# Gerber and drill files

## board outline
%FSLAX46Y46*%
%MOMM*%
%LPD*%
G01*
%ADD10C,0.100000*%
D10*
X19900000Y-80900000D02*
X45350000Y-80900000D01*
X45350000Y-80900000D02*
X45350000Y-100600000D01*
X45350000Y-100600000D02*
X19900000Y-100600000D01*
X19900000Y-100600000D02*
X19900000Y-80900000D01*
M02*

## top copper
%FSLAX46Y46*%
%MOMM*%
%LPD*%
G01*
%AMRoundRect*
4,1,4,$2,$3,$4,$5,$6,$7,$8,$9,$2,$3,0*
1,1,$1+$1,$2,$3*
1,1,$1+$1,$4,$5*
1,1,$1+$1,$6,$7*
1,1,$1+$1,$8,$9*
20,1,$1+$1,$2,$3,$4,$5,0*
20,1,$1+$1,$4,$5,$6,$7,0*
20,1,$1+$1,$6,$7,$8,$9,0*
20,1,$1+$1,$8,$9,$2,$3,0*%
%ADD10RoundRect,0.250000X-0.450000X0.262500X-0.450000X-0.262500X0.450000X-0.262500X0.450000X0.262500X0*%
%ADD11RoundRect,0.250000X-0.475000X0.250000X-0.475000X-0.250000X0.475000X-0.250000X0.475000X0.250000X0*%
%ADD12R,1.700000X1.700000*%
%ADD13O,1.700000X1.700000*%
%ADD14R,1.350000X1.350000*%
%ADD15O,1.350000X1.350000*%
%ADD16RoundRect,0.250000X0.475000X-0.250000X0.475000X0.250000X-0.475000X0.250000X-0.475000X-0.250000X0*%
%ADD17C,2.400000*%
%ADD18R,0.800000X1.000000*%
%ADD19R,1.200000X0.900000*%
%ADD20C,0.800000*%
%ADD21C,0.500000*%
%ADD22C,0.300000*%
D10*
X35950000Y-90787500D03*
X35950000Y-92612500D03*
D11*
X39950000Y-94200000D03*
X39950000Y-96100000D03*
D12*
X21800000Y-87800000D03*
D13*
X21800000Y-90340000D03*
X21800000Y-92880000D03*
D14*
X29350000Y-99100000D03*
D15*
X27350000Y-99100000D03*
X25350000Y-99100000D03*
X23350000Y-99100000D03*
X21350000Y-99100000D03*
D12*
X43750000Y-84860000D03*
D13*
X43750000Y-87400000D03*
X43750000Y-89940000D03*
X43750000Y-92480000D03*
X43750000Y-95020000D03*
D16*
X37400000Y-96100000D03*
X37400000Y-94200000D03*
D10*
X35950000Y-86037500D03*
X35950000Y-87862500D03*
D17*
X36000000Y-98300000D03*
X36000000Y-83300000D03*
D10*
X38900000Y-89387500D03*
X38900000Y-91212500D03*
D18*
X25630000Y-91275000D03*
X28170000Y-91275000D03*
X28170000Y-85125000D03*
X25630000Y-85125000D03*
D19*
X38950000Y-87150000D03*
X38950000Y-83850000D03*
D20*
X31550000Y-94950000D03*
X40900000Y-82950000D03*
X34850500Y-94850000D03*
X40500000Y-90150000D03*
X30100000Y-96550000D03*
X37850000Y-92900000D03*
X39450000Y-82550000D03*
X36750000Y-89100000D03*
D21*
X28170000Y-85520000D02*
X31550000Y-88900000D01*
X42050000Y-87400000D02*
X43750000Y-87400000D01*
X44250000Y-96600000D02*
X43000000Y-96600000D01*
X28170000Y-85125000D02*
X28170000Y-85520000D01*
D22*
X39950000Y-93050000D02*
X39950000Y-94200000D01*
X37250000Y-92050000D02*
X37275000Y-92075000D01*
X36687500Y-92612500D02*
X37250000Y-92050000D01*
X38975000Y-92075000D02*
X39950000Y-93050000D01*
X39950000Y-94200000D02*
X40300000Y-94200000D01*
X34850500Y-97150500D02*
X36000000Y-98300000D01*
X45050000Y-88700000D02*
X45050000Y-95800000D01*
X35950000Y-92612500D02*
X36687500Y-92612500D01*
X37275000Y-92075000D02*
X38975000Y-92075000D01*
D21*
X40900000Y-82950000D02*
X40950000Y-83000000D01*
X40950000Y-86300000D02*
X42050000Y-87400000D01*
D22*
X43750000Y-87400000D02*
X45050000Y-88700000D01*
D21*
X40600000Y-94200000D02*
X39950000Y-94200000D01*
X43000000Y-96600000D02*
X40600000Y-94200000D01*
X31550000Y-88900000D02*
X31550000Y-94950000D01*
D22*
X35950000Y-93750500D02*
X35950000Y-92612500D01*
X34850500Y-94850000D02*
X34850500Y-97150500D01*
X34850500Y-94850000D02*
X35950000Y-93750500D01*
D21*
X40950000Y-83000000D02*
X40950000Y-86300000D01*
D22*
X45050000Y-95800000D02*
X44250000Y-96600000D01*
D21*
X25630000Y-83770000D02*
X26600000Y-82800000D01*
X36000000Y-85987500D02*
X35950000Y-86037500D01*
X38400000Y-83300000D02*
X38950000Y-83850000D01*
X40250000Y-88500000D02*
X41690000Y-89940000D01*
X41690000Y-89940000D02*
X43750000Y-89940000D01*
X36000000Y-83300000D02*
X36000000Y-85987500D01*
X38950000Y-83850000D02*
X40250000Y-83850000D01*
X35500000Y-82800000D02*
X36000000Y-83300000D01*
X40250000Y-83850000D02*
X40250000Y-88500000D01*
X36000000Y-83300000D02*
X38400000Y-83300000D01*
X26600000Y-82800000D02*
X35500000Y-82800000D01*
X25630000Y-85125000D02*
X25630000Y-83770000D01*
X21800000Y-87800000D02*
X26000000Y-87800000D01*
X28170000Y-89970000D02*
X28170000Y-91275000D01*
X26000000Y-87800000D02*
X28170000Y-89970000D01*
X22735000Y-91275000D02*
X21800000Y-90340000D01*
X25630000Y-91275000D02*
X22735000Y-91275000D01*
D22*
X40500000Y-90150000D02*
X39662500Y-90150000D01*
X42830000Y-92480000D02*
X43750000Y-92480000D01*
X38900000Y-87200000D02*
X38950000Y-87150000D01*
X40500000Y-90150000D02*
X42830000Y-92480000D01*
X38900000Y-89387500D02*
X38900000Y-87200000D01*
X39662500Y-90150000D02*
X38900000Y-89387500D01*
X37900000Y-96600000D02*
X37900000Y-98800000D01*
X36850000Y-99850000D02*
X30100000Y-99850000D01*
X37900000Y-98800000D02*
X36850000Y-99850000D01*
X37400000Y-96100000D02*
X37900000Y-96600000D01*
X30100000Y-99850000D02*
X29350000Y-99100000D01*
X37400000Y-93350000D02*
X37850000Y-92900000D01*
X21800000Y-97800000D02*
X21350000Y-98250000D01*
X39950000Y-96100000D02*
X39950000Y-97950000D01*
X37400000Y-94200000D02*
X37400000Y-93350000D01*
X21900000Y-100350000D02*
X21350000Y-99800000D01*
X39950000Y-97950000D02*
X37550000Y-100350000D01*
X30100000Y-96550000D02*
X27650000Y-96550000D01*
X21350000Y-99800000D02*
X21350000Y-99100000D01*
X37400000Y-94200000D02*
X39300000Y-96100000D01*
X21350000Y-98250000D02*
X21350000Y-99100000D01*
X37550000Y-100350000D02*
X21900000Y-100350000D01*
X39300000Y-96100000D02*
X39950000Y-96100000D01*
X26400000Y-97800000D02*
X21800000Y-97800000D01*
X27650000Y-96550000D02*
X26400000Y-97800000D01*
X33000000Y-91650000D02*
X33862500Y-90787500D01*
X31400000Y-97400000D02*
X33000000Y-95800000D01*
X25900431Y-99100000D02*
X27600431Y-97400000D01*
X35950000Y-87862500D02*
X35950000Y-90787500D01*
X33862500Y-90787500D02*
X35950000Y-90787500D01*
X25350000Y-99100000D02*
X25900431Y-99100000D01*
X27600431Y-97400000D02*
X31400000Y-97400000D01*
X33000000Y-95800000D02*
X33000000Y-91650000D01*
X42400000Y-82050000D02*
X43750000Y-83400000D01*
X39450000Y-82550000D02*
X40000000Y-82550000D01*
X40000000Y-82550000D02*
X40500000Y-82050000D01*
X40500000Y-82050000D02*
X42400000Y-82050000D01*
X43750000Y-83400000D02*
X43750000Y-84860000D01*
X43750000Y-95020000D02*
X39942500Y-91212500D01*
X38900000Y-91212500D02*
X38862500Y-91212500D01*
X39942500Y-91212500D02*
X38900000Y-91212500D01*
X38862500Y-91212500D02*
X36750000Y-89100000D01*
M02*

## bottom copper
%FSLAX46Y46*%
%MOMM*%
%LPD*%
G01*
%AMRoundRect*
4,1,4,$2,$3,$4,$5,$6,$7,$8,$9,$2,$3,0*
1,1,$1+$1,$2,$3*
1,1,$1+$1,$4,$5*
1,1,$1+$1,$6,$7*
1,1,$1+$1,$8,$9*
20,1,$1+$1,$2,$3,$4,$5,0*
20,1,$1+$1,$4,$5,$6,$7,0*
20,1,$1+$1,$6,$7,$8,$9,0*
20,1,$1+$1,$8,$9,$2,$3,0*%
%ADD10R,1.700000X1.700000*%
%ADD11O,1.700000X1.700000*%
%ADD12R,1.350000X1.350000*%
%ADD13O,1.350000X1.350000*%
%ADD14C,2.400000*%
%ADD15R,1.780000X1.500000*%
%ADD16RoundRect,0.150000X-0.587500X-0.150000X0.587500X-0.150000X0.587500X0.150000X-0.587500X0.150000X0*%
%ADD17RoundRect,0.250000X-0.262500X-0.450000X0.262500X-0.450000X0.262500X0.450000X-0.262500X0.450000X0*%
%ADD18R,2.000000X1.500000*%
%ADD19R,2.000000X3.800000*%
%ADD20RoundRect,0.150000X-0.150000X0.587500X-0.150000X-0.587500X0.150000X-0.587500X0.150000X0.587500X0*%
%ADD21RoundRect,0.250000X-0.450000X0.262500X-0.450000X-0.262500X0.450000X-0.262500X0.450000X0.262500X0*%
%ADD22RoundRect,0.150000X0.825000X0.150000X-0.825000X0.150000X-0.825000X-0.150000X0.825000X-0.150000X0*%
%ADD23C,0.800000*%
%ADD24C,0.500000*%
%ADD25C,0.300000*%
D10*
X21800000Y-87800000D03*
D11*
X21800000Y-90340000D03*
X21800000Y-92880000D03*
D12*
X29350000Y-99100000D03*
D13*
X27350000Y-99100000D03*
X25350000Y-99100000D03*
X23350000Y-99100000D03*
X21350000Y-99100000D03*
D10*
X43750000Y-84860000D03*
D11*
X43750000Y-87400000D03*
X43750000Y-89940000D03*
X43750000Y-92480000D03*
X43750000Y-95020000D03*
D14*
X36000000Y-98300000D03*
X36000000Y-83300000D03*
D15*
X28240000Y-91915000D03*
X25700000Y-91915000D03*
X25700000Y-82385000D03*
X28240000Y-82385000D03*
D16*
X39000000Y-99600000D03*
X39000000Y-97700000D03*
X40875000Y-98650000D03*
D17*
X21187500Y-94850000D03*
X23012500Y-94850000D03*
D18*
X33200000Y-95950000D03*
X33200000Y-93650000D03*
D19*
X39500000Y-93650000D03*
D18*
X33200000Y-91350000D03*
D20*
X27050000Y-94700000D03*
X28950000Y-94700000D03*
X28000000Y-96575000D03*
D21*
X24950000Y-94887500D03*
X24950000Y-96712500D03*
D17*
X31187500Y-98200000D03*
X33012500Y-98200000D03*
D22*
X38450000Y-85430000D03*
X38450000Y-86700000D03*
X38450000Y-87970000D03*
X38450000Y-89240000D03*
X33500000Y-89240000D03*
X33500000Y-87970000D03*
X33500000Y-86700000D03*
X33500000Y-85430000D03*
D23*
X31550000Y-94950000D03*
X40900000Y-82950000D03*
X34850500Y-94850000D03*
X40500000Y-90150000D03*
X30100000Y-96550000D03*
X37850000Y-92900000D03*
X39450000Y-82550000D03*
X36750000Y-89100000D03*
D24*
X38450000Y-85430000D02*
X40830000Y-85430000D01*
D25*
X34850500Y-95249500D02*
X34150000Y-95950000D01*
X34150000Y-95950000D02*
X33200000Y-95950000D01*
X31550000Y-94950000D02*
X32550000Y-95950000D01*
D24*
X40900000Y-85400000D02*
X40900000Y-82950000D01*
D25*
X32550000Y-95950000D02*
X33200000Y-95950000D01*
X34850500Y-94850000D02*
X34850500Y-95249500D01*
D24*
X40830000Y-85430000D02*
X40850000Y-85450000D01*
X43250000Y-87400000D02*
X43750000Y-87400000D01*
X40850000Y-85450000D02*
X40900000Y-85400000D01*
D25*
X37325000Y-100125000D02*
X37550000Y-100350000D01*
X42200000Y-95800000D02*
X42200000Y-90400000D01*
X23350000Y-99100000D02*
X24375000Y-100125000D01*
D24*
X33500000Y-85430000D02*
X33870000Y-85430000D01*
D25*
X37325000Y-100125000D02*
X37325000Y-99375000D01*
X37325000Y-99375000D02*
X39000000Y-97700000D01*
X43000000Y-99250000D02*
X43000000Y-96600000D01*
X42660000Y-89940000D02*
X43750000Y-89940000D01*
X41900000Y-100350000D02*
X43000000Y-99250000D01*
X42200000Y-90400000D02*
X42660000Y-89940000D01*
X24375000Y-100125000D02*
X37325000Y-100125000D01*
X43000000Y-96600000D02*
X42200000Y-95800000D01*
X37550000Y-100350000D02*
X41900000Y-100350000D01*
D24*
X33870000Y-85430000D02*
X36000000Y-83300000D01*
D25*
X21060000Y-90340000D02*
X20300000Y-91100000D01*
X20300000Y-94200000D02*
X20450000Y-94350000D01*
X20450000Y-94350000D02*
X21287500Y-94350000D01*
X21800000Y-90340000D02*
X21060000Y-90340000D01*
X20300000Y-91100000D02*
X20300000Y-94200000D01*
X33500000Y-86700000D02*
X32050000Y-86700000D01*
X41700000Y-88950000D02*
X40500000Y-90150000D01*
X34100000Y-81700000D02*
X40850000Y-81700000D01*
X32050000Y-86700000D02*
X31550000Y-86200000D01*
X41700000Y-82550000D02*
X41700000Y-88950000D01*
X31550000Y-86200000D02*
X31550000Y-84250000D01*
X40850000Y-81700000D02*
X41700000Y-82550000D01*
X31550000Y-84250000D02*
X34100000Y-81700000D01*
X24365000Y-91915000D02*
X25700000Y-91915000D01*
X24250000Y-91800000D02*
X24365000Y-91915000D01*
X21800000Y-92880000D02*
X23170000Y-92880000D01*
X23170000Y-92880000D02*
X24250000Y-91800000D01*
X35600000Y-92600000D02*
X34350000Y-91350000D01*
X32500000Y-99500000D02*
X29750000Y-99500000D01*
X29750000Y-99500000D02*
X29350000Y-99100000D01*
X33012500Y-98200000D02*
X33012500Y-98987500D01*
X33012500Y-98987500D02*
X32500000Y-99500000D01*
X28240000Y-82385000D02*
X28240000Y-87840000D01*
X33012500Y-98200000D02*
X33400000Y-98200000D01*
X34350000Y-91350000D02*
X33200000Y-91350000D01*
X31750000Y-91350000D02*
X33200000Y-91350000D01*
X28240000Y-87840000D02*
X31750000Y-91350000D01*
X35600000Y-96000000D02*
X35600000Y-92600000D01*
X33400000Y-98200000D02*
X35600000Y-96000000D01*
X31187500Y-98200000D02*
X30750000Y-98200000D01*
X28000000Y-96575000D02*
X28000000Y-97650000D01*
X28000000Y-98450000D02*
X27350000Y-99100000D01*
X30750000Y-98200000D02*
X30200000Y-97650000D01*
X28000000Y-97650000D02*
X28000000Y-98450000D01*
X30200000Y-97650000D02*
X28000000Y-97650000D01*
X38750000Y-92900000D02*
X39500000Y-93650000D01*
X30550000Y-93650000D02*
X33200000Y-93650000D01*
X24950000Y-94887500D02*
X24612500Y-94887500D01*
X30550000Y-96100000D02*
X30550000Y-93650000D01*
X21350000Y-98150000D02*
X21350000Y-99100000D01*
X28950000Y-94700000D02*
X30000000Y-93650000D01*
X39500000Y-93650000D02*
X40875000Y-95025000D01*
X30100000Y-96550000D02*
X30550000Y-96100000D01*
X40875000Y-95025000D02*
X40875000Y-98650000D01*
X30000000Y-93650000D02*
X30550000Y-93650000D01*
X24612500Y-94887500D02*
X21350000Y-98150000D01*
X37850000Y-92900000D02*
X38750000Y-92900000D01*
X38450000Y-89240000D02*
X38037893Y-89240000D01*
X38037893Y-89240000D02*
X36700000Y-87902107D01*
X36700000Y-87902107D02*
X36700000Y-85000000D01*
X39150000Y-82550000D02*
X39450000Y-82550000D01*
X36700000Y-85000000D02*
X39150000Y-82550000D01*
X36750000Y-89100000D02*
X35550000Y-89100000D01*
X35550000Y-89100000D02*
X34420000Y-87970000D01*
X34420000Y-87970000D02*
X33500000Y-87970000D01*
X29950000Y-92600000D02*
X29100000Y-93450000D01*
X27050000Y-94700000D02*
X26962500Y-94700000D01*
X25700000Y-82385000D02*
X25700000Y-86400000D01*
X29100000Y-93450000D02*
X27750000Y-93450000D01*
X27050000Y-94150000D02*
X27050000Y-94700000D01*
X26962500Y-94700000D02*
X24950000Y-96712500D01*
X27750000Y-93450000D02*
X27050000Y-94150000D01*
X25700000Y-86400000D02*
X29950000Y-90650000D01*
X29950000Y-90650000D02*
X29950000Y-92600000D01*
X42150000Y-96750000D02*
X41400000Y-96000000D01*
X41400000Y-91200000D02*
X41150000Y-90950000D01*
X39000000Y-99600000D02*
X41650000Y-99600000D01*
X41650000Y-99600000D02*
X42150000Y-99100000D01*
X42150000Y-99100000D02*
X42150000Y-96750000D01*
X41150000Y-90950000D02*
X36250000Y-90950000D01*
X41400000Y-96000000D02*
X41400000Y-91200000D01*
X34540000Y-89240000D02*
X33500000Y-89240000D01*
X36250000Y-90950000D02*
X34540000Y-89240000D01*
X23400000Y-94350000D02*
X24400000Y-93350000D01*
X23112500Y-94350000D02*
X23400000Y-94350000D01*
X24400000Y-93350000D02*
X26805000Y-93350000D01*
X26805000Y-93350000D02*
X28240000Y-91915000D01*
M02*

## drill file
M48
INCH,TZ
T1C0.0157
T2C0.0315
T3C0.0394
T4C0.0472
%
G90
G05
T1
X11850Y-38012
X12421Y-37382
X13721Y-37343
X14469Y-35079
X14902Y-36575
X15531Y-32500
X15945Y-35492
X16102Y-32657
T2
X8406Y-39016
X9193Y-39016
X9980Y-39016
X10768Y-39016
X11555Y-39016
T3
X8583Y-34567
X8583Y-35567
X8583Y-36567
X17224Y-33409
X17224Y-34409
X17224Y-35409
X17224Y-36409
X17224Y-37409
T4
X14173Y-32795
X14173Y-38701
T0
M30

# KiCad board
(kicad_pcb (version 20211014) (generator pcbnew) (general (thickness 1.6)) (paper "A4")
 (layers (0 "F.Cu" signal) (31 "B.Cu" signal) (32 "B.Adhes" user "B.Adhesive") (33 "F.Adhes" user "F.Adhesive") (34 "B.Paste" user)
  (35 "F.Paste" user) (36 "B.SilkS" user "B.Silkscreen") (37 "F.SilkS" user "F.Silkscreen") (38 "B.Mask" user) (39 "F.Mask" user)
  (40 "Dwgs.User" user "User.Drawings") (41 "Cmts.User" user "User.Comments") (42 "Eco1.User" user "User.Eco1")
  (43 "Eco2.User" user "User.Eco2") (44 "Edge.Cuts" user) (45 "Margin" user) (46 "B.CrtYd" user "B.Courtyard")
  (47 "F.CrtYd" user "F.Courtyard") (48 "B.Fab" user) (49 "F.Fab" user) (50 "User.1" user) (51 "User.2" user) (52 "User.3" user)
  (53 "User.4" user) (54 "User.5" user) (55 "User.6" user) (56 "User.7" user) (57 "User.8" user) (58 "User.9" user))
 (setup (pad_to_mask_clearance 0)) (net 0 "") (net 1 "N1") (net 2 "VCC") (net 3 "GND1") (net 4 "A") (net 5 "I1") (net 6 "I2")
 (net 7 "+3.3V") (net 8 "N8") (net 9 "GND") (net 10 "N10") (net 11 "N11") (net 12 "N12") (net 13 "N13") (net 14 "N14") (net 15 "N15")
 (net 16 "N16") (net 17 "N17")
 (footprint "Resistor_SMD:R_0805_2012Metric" (layer "F.Cu") (at 35.95 91.7 -90)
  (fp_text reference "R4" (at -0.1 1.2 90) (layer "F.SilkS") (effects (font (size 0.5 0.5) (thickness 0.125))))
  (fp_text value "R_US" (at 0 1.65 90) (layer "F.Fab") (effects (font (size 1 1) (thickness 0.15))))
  (pad "1" smd roundrect (at -0.9125 0 270) (size 1.025 1.4) (layers "F.Cu" "F.Paste" "F.Mask") (roundrect_rratio 0.243902439) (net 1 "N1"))
  (pad "2" smd roundrect (at 0.9125 0 270) (size 1.025 1.4) (layers "F.Cu" "F.Paste" "F.Mask") (roundrect_rratio 0.243902439) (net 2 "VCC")))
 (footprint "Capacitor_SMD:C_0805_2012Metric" (layer "F.Cu") (at 39.95 95.15 -90)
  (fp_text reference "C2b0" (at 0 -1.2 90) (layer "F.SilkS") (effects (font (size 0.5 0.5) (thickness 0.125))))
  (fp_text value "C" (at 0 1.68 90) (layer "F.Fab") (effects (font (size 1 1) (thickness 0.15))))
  (pad "1" smd roundrect (at -0.95 0 270) (size 1 1.45) (layers "F.Cu" "F.Paste" "F.Mask") (roundrect_rratio 0.25) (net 2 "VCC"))
  (pad "2" smd roundrect (at 0.95 0 270) (size 1 1.45) (layers "F.Cu" "F.Paste" "F.Mask") (roundrect_rratio 0.25) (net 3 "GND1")))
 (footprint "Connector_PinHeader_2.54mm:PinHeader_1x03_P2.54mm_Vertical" (layer "F.Cu") (at 21.8 87.8)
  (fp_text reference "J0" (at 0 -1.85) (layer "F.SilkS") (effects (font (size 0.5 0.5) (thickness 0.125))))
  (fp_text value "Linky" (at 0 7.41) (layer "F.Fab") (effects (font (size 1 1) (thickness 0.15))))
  (pad "1" thru_hole rect (at 0 0) (size 1.7 1.7) (drill 1) (layers *.Cu *.Mask) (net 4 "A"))
  (pad "2" thru_hole oval (at 0 2.54) (size 1.7 1.7) (drill 1) (layers *.Cu *.Mask) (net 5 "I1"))
  (pad "3" thru_hole oval (at 0 5.08) (size 1.7 1.7) (drill 1) (layers *.Cu *.Mask) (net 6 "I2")))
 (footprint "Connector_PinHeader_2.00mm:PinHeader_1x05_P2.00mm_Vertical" (layer "F.Cu") (at 29.35 99.1 -90)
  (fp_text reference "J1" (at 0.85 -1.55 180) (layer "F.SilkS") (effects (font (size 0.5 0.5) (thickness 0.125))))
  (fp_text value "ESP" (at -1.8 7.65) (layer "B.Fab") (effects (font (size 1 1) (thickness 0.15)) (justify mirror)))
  (pad "1" thru_hole rect (at 0 0 270) (size 1.35 1.35) (drill 0.8) (layers *.Cu *.Mask) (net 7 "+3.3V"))
  (pad "2" thru_hole oval (at 0 2 270) (size 1.35 1.35) (drill 0.8) (layers *.Cu *.Mask) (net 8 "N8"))
  (pad "3" thru_hole oval (at 0 4 270) (size 1.35 1.35) (drill 0.8) (layers *.Cu *.Mask) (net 1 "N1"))
  (pad "4" thru_hole oval (at 0 6 270) (size 1.35 1.35) (drill 0.8) (layers *.Cu *.Mask) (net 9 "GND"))
  (pad "5" thru_hole oval (at 0 8 270) (size 1.35 1.35) (drill 0.8) (layers *.Cu *.Mask) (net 3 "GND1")))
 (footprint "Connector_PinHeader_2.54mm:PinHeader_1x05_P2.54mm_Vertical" (layer "F.Cu") (at 43.75 84.86)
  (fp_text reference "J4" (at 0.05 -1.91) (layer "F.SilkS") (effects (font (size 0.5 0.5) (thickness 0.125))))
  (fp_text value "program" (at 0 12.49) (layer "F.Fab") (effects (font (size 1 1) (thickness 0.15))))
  (pad "1" thru_hole rect (at 0 0) (size 1.7 1.7) (drill 1) (layers *.Cu *.Mask) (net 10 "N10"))
  (pad "2" thru_hole oval (at 0 2.54) (size 1.7 1.7) (drill 1) (layers *.Cu *.Mask) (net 2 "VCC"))
  (pad "3" thru_hole oval (at 0 5.08) (size 1.7 1.7) (drill 1) (layers *.Cu *.Mask) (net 9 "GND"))
  (pad "4" thru_hole oval (at 0 7.62) (size 1.7 1.7) (drill 1) (layers *.Cu *.Mask) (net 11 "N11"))
  (pad "5" thru_hole oval (at 0 10.16) (size 1.7 1.7) (drill 1) (layers *.Cu *.Mask) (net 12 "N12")))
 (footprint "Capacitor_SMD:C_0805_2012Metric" (layer "F.Cu") (at 37.4 95.15 90)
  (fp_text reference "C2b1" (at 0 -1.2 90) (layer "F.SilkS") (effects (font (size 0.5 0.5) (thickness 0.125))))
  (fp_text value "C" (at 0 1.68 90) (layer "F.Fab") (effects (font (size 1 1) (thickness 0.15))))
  (pad "1" smd roundrect (at -0.95 0 90) (size 1 1.45) (layers "F.Cu" "F.Paste" "F.Mask") (roundrect_rratio 0.25) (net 7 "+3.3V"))
  (pad "2" smd roundrect (at 0.95 0 90) (size 1 1.45) (layers "F.Cu" "F.Paste" "F.Mask") (roundrect_rratio 0.25) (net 3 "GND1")))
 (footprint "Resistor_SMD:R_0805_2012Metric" (layer "F.Cu") (at 35.95 86.95 -90)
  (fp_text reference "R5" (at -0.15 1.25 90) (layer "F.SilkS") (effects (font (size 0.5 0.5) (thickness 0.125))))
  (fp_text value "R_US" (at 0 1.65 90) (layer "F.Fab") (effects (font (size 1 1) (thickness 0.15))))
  (pad "1" smd roundrect (at -0.9125 0 270) (size 1.025 1.4) (layers "F.Cu" "F.Paste" "F.Mask") (roundrect_rratio 0.243902439) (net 9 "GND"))
  (pad "2" smd roundrect (at 0.9125 0 270) (size 1.025 1.4) (layers "F.Cu" "F.Paste" "F.Mask") (roundrect_rratio 0.243902439) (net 1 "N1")))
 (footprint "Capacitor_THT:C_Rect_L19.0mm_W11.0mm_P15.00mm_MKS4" (layer "F.Cu") (at 36 98.3 90)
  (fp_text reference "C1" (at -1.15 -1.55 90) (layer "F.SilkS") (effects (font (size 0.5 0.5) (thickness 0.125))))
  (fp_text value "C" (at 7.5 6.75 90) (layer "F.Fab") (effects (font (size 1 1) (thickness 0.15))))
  (pad "1" thru_hole circle (at 0 0 90) (size 2.4 2.4) (drill 1.2) (layers *.Cu *.Mask) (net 2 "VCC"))
  (pad "2" thru_hole circle (at 15 0 90) (size 2.4 2.4) (drill 1.2) (layers *.Cu *.Mask) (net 9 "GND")))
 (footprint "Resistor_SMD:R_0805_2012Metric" (layer "F.Cu") (at 38.9 90.3 -90)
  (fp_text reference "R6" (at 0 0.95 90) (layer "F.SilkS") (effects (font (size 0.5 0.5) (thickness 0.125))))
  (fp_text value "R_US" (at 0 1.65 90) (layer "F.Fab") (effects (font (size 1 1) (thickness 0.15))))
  (pad "1" smd roundrect (at -0.9125 0 270) (size 1.025 1.4) (layers "F.Cu" "F.Paste" "F.Mask") (roundrect_rratio 0.243902439)
   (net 11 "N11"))
  (pad "2" smd roundrect (at 0.9125 0 270) (size 1.025 1.4) (layers "F.Cu" "F.Paste" "F.Mask") (roundrect_rratio 0.243902439) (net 12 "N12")))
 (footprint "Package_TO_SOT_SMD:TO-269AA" (layer "F.Cu") (at 26.9 88.2 90)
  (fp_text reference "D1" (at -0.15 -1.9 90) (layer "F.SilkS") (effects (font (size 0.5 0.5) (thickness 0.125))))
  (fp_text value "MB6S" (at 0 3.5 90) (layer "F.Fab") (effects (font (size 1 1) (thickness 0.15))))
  (pad "1" smd rect (at -3.075 -1.27 90) (size 1 0.8) (layers "F.Cu" "F.Paste" "F.Mask") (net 5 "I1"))
  (pad "2" smd rect (at -3.075 1.27 90) (size 1 0.8) (layers "F.Cu" "F.Paste" "F.Mask") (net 4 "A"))
  (pad "3" smd rect (at 3.075 1.27 90) (size 1 0.8) (layers "F.Cu" "F.Paste" "F.Mask") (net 2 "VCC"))
  (pad "4" smd rect (at 3.075 -1.27 90) (size 1 0.8) (layers "F.Cu" "F.Paste" "F.Mask") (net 9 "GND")))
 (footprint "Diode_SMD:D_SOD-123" (layer "F.Cu") (at 38.95 85.5 90)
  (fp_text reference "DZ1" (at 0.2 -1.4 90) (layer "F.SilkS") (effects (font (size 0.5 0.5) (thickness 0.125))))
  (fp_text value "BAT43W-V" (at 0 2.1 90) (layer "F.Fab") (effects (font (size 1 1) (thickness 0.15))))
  (pad "1" smd rect (at -1.65 0 90) (size 0.9 1.2) (layers "F.Cu" "F.Paste" "F.Mask") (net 11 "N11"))
  (pad "2" smd rect (at 1.65 0 90) (size 0.9 1.2) (layers "F.Cu" "F.Paste" "F.Mask") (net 9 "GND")))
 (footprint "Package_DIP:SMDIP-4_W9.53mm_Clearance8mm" (layer "B.Cu") (at 26.97 87.15 90)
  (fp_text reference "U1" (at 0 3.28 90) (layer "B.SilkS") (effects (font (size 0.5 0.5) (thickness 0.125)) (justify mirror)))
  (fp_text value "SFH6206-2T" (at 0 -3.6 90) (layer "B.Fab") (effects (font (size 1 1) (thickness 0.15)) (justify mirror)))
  (pad "1" smd rect (at -4.765 1.27 90) (size 1.5 1.78) (layers "B.Cu" "B.Paste" "B.Mask") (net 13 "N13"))
  (pad "2" smd rect (at -4.765 -1.27 90) (size 1.5 1.78) (layers "B.Cu" "B.Paste" "B.Mask") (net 6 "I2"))
  (pad "3" smd rect (at 4.765 -1.27 90) (size 1.5 1.78) (layers "B.Cu" "B.Paste" "B.Mask") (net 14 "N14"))
  (pad "4" smd rect (at 4.765 1.27 90) (size 1.5 1.78) (layers "B.Cu" "B.Paste" "B.Mask") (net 7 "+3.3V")))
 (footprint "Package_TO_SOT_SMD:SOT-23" (layer "B.Cu") (at 39.9375 98.65)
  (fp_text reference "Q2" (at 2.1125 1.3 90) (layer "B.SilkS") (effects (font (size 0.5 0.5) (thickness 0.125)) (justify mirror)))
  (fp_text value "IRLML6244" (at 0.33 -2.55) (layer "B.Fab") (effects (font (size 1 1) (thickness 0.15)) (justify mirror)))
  (pad "1" smd roundrect (at -0.9375 0.95) (size 1.475 0.6) (layers "B.Cu" "B.Paste" "B.Mask") (roundrect_rratio 0.25) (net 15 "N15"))
  (pad "2" smd roundrect (at -0.9375 -0.95) (size 1.475 0.6) (layers "B.Cu" "B.Paste" "B.Mask") (roundrect_rratio 0.25) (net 9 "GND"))
  (pad "3" smd roundrect (at 0.9375 0) (size 1.475 0.6) (layers "B.Cu" "B.Paste" "B.Mask") (roundrect_rratio 0.25) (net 3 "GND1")))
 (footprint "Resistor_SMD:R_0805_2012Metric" (layer "B.Cu") (at 22.1 94.85)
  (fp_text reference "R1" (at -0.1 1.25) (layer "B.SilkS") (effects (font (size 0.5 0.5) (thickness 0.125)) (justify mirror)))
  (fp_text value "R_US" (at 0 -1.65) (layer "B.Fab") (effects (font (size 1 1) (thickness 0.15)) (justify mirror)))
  (pad "1" smd roundrect (at -0.9125 0) (size 1.025 1.4) (layers "B.Cu" "B.Paste" "B.Mask") (roundrect_rratio 0.243902439) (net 5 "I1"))
  (pad "2" smd roundrect (at 0.9125 0) (size 1.025 1.4) (layers "B.Cu" "B.Paste" "B.Mask") (roundrect_rratio 0.243902439) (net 13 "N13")))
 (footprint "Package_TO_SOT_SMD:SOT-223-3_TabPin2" (layer "B.Cu") (at 36.35 93.65)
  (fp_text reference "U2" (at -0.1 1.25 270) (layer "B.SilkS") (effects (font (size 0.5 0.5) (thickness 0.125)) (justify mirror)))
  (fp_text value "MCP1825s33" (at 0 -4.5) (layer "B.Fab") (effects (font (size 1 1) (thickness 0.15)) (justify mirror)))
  (pad "1" smd rect (at -3.15 2.3) (size 2 1.5) (layers "B.Cu" "B.Paste" "B.Mask") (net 2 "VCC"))
  (pad "2" smd rect (at -3.15 0) (size 2 1.5) (layers "B.Cu" "B.Paste" "B.Mask") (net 3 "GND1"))
  (pad "2" smd rect (at 3.15 0) (size 2 3.8) (layers "B.Cu" "B.Paste" "B.Mask") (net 3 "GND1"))
  (pad "3" smd rect (at -3.15 -2.3) (size 2 1.5) (layers "B.Cu" "B.Paste" "B.Mask") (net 7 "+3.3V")))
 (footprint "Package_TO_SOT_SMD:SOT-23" (layer "B.Cu") (at 28 95.6375 -90)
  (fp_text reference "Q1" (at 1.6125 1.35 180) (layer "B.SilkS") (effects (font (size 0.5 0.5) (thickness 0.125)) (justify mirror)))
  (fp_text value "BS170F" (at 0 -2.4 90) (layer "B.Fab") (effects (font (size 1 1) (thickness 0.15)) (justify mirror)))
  (pad "1" smd roundrect (at -0.9375 0.95 270) (size 1.475 0.6) (layers "B.Cu" "B.Paste" "B.Mask") (roundrect_rratio 0.25) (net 14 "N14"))
  (pad "2" smd roundrect (at -0.9375 -0.95 270) (size 1.475 0.6) (layers "B.Cu" "B.Paste" "B.Mask") (roundrect_rratio 0.25) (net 3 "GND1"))
  (pad "3" smd roundrect (at 0.9375 0 270) (size 1.475 0.6) (layers "B.Cu" "B.Paste" "B.Mask") (roundrect_rratio 0.25) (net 8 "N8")))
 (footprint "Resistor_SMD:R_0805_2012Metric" (layer "B.Cu") (at 24.95 95.8 -90)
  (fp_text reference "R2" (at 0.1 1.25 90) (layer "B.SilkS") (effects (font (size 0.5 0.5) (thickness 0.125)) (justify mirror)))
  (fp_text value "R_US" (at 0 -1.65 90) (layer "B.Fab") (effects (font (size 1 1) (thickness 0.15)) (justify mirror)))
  (pad "1" smd roundrect (at -0.9125 0 270) (size 1.025 1.4) (layers "B.Cu" "B.Paste" "B.Mask") (roundrect_rratio 0.243902439)
   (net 3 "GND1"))
  (pad "2" smd roundrect (at 0.9125 0 270) (size 1.025 1.4) (layers "B.Cu" "B.Paste" "B.Mask") (roundrect_rratio 0.243902439) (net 14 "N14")))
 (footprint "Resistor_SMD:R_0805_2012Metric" (layer "B.Cu") (at 32.1 98.2)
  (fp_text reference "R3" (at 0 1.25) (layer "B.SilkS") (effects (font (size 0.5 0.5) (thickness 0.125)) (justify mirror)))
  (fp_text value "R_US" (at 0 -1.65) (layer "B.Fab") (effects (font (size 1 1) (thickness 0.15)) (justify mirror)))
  (pad "1" smd roundrect (at -0.9125 0) (size 1.025 1.4) (layers "B.Cu" "B.Paste" "B.Mask") (roundrect_rratio 0.243902439) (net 8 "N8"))
  (pad "2" smd roundrect (at 0.9125 0) (size 1.025 1.4) (layers "B.Cu" "B.Paste" "B.Mask") (roundrect_rratio 0.243902439) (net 7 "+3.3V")))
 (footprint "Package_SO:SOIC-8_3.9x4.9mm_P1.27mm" (layer "B.Cu") (at 35.975 87.335 180)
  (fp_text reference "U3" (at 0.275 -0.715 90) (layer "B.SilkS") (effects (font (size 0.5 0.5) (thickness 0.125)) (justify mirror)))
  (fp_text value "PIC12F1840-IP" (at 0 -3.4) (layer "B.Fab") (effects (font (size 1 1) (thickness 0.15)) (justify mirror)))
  (pad "1" smd roundrect (at -2.475 1.905 180) (size 1.95 0.6) (layers "B.Cu" "B.Paste" "B.Mask") (roundrect_rratio 0.25) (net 2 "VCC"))
  (pad "2" smd roundrect (at -2.475 0.635 180) (size 1.95 0.6) (layers "B.Cu" "B.Paste" "B.Mask") (roundrect_rratio 0.25) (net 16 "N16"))
  (pad "3" smd roundrect (at -2.475 -0.635 180) (size 1.95 0.6) (layers "B.Cu" "B.Paste" "B.Mask") (roundrect_rratio 0.25) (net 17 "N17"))
  (pad "4" smd roundrect (at -2.475 -1.905 180) (size 1.95 0.6) (layers "B.Cu" "B.Paste" "B.Mask") (roundrect_rratio 0.25) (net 10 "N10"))
  (pad "5" smd roundrect (at 2.475 -1.905 180) (size 1.95 0.6) (layers "B.Cu" "B.Paste" "B.Mask") (roundrect_rratio 0.25) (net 15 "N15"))
  (pad "6" smd roundrect (at 2.475 -0.635 180) (size 1.95 0.6) (layers "B.Cu" "B.Paste" "B.Mask") (roundrect_rratio 0.25) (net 12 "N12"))
  (pad "7" smd roundrect (at 2.475 0.635 180) (size 1.95 0.6) (layers "B.Cu" "B.Paste" "B.Mask") (roundrect_rratio 0.25) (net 11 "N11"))
  (pad "8" smd roundrect (at 2.475 1.905 180) (size 1.95 0.6) (layers "B.Cu" "B.Paste" "B.Mask") (roundrect_rratio 0.25) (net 9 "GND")))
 (gr_rect (start 19.9 80.9) (end 45.35 100.6) (layer "Edge.Cuts") (width 0.1) (fill none))
 (segment (start 28.17 85.52) (end 31.55 88.9) (width 0.5) (layer "F.Cu") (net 2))
 (segment (start 42.05 87.4) (end 43.75 87.4) (width 0.5) (layer "F.Cu") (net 2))
 (segment (start 44.25 96.6) (end 43 96.6) (width 0.5) (layer "F.Cu") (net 2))
 (segment (start 28.17 85.125) (end 28.17 85.52) (width 0.5) (layer "F.Cu") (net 2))
 (segment (start 39.95 93.05) (end 39.95 94.2) (width 0.3) (layer "F.Cu") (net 2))
 (segment (start 37.25 92.05) (end 37.275 92.075) (width 0.3) (layer "F.Cu") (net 2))
 (segment (start 36.6875 92.6125) (end 37.25 92.05) (width 0.3) (layer "F.Cu") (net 2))
 (segment (start 38.975 92.075) (end 39.95 93.05) (width 0.3) (layer "F.Cu") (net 2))
 (segment (start 39.95 94.2) (end 40.3 94.2) (width 0.3) (layer "F.Cu") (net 2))
 (segment (start 34.8505 97.1505) (end 36 98.3) (width 0.3) (layer "F.Cu") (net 2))
 (segment (start 45.05 88.7) (end 45.05 95.8) (width 0.3) (layer "F.Cu") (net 2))
 (segment (start 35.95 92.6125) (end 36.6875 92.6125) (width 0.3) (layer "F.Cu") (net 2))
 (segment (start 37.275 92.075) (end 38.975 92.075) (width 0.3) (layer "F.Cu") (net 2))
 (segment (start 40.9 82.95) (end 40.95 83) (width 0.5) (layer "F.Cu") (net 2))
 (segment (start 40.95 86.3) (end 42.05 87.4) (width 0.5) (layer "F.Cu") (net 2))
 (segment (start 43.75 87.4) (end 45.05 88.7) (width 0.3) (layer "F.Cu") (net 2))
 (segment (start 40.6 94.2) (end 39.95 94.2) (width 0.5) (layer "F.Cu") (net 2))
 (segment (start 43 96.6) (end 40.6 94.2) (width 0.5) (layer "F.Cu") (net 2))
 (segment (start 31.55 88.9) (end 31.55 94.95) (width 0.5) (layer "F.Cu") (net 2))
 (segment (start 35.95 93.7505) (end 35.95 92.6125) (width 0.3) (layer "F.Cu") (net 2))
 (segment (start 34.8505 94.85) (end 34.8505 97.1505) (width 0.3) (layer "F.Cu") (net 2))
 (segment (start 34.8505 94.85) (end 35.95 93.7505) (width 0.3) (layer "F.Cu") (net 2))
 (segment (start 40.95 83) (end 40.95 86.3) (width 0.5) (layer "F.Cu") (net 2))
 (segment (start 45.05 95.8) (end 44.25 96.6) (width 0.3) (layer "F.Cu") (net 2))
 (via (at 31.55 94.95) (size 0.8) (drill 0.4) (layers "F.Cu" "B.Cu") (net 2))
 (via (at 40.9 82.95) (size 0.8) (drill 0.4) (layers "F.Cu" "B.Cu") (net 2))
 (via (at 34.8505 94.85) (size 0.8) (drill 0.4) (layers "F.Cu" "B.Cu") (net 2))
 (segment (start 38.45 85.43) (end 40.83 85.43) (width 0.5) (layer "B.Cu") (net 2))
 (segment (start 34.8505 95.2495) (end 34.15 95.95) (width 0.3) (layer "B.Cu") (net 2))
 (segment (start 34.15 95.95) (end 33.2 95.95) (width 0.3) (layer "B.Cu") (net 2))
 (segment (start 31.55 94.95) (end 32.55 95.95) (width 0.3) (layer "B.Cu") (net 2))
 (segment (start 40.9 85.4) (end 40.9 82.95) (width 0.5) (layer "B.Cu") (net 2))
 (segment (start 32.55 95.95) (end 33.2 95.95) (width 0.3) (layer "B.Cu") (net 2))
 (segment (start 34.8505 94.85) (end 34.8505 95.2495) (width 0.3) (layer "B.Cu") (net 2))
 (segment (start 40.83 85.43) (end 40.85 85.45) (width 0.5) (layer "B.Cu") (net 2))
 (segment (start 43.25 87.4) (end 43.75 87.4) (width 0.5) (layer "B.Cu") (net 2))
 (segment (start 40.85 85.45) (end 40.9 85.4) (width 0.5) (layer "B.Cu") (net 2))
 (segment (start 25.63 83.77) (end 26.6 82.8) (width 0.5) (layer "F.Cu") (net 9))
 (segment (start 36 85.9875) (end 35.95 86.0375) (width 0.5) (layer "F.Cu") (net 9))
 (segment (start 38.4 83.3) (end 38.95 83.85) (width 0.5) (layer "F.Cu") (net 9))
 (segment (start 40.25 88.5) (end 41.69 89.94) (width 0.5) (layer "F.Cu") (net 9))
 (segment (start 41.69 89.94) (end 43.75 89.94) (width 0.5) (layer "F.Cu") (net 9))
 (segment (start 36 83.3) (end 36 85.9875) (width 0.5) (layer "F.Cu") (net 9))
 (segment (start 38.95 83.85) (end 40.25 83.85) (width 0.5) (layer "F.Cu") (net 9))
 (segment (start 35.5 82.8) (end 36 83.3) (width 0.5) (layer "F.Cu") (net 9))
 (segment (start 40.25 83.85) (end 40.25 88.5) (width 0.5) (layer "F.Cu") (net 9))
 (segment (start 36 83.3) (end 38.4 83.3) (width 0.5) (layer "F.Cu") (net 9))
 (segment (start 26.6 82.8) (end 35.5 82.8) (width 0.5) (layer "F.Cu") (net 9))
 (segment (start 25.63 85.125) (end 25.63 83.77) (width 0.5) (layer "F.Cu") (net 9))
 (segment (start 37.325 100.125) (end 37.55 100.35) (width 0.3) (layer "B.Cu") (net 9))
 (segment (start 42.2 95.8) (end 42.2 90.4) (width 0.3) (layer "B.Cu") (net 9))
 (segment (start 23.35 99.1) (end 24.375 100.125) (width 0.3) (layer "B.Cu") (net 9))
 (segment (start 33.5 85.43) (end 33.87 85.43) (width 0.5) (layer "B.Cu") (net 9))
 (segment (start 37.325 100.125) (end 37.325 99.375) (width 0.3) (layer "B.Cu") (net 9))
 (segment (start 37.325 99.375) (end 39 97.7) (width 0.3) (layer "B.Cu") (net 9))
 (segment (start 43 99.25) (end 43 96.6) (width 0.3) (layer "B.Cu") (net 9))
 (segment (start 42.66 89.94) (end 43.75 89.94) (width 0.3) (layer "B.Cu") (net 9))
 (segment (start 41.9 100.35) (end 43 99.25) (width 0.3) (layer "B.Cu") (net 9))
 (segment (start 42.2 90.4) (end 42.66 89.94) (width 0.3) (layer "B.Cu") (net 9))
 (segment (start 24.375 100.125) (end 37.325 100.125) (width 0.3) (layer "B.Cu") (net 9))
 (segment (start 43 96.6) (end 42.2 95.8) (width 0.3) (layer "B.Cu") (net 9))
 (segment (start 37.55 100.35) (end 41.9 100.35) (width 0.3) (layer "B.Cu") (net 9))
 (segment (start 33.87 85.43) (end 36 83.3) (width 0.5) (layer "B.Cu") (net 9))
 (segment (start 21.8 87.8) (end 26 87.8) (width 0.5) (layer "F.Cu") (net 4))
 (segment (start 28.17 89.97) (end 28.17 91.275) (width 0.5) (layer "F.Cu") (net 4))
 (segment (start 26 87.8) (end 28.17 89.97) (width 0.5) (layer "F.Cu") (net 4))
 (segment (start 22.735 91.275) (end 21.8 90.34) (width 0.5) (layer "F.Cu") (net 5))
 (segment (start 25.63 91.275) (end 22.735 91.275) (width 0.5) (layer "F.Cu") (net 5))
 (segment (start 21.06 90.34) (end 20.3 91.1) (width 0.3) (layer "B.Cu") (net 5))
 (segment (start 20.3 94.2) (end 20.45 94.35) (width 0.3) (layer "B.Cu") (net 5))
 (segment (start 20.45 94.35) (end 21.2875 94.35) (width 0.3) (layer "B.Cu") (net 5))
 (segment (start 21.8 90.34) (end 21.06 90.34) (width 0.3) (layer "B.Cu") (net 5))
 (segment (start 20.3 91.1) (end 20.3 94.2) (width 0.3) (layer "B.Cu") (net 5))
 (segment (start 40.5 90.15) (end 39.6625 90.15) (width 0.3) (layer "F.Cu") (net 11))
 (segment (start 42.83 92.48) (end 43.75 92.48) (width 0.3) (layer "F.Cu") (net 11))
 (segment (start 38.9 87.2) (end 38.95 87.15) (width 0.3) (layer "F.Cu") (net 11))
 (segment (start 40.5 90.15) (end 42.83 92.48) (width 0.3) (layer "F.Cu") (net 11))
 (segment (start 38.9 89.3875) (end 38.9 87.2) (width 0.3) (layer "F.Cu") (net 11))
 (segment (start 39.6625 90.15) (end 38.9 89.3875) (width 0.3) (layer "F.Cu") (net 11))
 (via (at 40.5 90.15) (size 0.8) (drill 0.4) (layers "F.Cu" "B.Cu") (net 11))
 (segment (start 33.5 86.7) (end 32.05 86.7) (width 0.3) (layer "B.Cu") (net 11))
 (segment (start 41.7 88.95) (end 40.5 90.15) (width 0.3) (layer "B.Cu") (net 11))
 (segment (start 34.1 81.7) (end 40.85 81.7) (width 0.3) (layer "B.Cu") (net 11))
 (segment (start 32.05 86.7) (end 31.55 86.2) (width 0.3) (layer "B.Cu") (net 11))
 (segment (start 41.7 82.55) (end 41.7 88.95) (width 0.3) (layer "B.Cu") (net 11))
 (segment (start 31.55 86.2) (end 31.55 84.25) (width 0.3) (layer "B.Cu") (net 11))
 (segment (start 40.85 81.7) (end 41.7 82.55) (width 0.3) (layer "B.Cu") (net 11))
 (segment (start 31.55 84.25) (end 34.1 81.7) (width 0.3) (layer "B.Cu") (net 11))
 (segment (start 24.365 91.915) (end 25.7 91.915) (width 0.3) (layer "B.Cu") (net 6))
 (segment (start 24.25 91.8) (end 24.365 91.915) (width 0.3) (layer "B.Cu") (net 6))
 (segment (start 21.8 92.88) (end 23.17 92.88) (width 0.3) (layer "B.Cu") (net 6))
 (segment (start 23.17 92.88) (end 24.25 91.8) (width 0.3) (layer "B.Cu") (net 6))
 (segment (start 37.9 96.6) (end 37.9 98.8) (width 0.3) (layer "F.Cu") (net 7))
 (segment (start 36.85 99.85) (end 30.1 99.85) (width 0.3) (layer "F.Cu") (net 7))
 (segment (start 37.9 98.8) (end 36.85 99.85) (width 0.3) (layer "F.Cu") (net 7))
 (segment (start 37.4 96.1) (end 37.9 96.6) (width 0.3) (layer "F.Cu") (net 7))
 (segment (start 30.1 99.85) (end 29.35 99.1) (width 0.3) (layer "F.Cu") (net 7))
 (segment (start 35.6 92.6) (end 34.35 91.35) (width 0.3) (layer "B.Cu") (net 7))
 (segment (start 32.5 99.5) (end 29.75 99.5) (width 0.3) (layer "B.Cu") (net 7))
 (segment (start 29.75 99.5) (end 29.35 99.1) (width 0.3) (layer "B.Cu") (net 7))
 (segment (start 33.0125 98.2) (end 33.0125 98.9875) (width 0.3) (layer "B.Cu") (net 7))
 (segment (start 33.0125 98.9875) (end 32.5 99.5) (width 0.3) (layer "B.Cu") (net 7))
 (segment (start 28.24 82.385) (end 28.24 87.84) (width 0.3) (layer "B.Cu") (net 7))
 (segment (start 33.0125 98.2) (end 33.4 98.2) (width 0.3) (layer "B.Cu") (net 7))
 (segment (start 34.35 91.35) (end 33.2 91.35) (width 0.3) (layer "B.Cu") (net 7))
 (segment (start 31.75 91.35) (end 33.2 91.35) (width 0.3) (layer "B.Cu") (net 7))
 (segment (start 28.24 87.84) (end 31.75 91.35) (width 0.3) (layer "B.Cu") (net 7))
 (segment (start 35.6 96) (end 35.6 92.6) (width 0.3) (layer "B.Cu") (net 7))
 (segment (start 33.4 98.2) (end 35.6 96) (width 0.3) (layer "B.Cu") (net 7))
 (segment (start 31.1875 98.2) (end 30.75 98.2) (width 0.3) (layer "B.Cu") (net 8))
 (segment (start 28 96.575) (end 28 97.65) (width 0.3) (layer "B.Cu") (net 8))
 (segment (start 28 98.45) (end 27.35 99.1) (width 0.3) (layer "B.Cu") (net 8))
 (segment (start 30.75 98.2) (end 30.2 97.65) (width 0.3) (layer "B.Cu") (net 8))
 (segment (start 28 97.65) (end 28 98.45) (width 0.3) (layer "B.Cu") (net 8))
 (segment (start 30.2 97.65) (end 28 97.65) (width 0.3) (layer "B.Cu") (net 8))
 (segment (start 37.4 93.35) (end 37.85 92.9) (width 0.3) (layer "F.Cu") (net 3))
 (segment (start 21.8 97.8) (end 21.35 98.25) (width 0.3) (layer "F.Cu") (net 3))
 (segment (start 39.95 96.1) (end 39.95 97.95) (width 0.3) (layer "F.Cu") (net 3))
 (segment (start 37.4 94.2) (end 37.4 93.35) (width 0.3) (layer "F.Cu") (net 3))
 (segment (start 21.9 100.35) (end 21.35 99.8) (width 0.3) (layer "F.Cu") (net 3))
 (segment (start 39.95 97.95) (end 37.55 100.35) (width 0.3) (layer "F.Cu") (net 3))
 (segment (start 30.1 96.55) (end 27.65 96.55) (width 0.3) (layer "F.Cu") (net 3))
 (segment (start 21.35 99.8) (end 21.35 99.1) (width 0.3) (layer "F.Cu") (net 3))
 (segment (start 37.4 94.2) (end 39.3 96.1) (width 0.3) (layer "F.Cu") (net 3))
 (segment (start 21.35 98.25) (end 21.35 99.1) (width 0.3) (layer "F.Cu") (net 3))
 (segment (start 37.55 100.35) (end 21.9 100.35) (width 0.3) (layer "F.Cu") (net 3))
 (segment (start 39.3 96.1) (end 39.95 96.1) (width 0.3) (layer "F.Cu") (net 3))
 (segment (start 26.4 97.8) (end 21.8 97.8) (width 0.3) (layer "F.Cu") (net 3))
 (segment (start 27.65 96.55) (end 26.4 97.8) (width 0.3) (layer "F.Cu") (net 3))
 (via (at 30.1 96.55) (size 0.8) (drill 0.4) (layers "F.Cu" "B.Cu") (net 3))
 (via (at 37.85 92.9) (size 0.8) (drill 0.4) (layers "F.Cu" "B.Cu") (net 3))
 (segment (start 38.75 92.9) (end 39.5 93.65) (width 0.3) (layer "B.Cu") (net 3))
 (segment (start 30.55 93.65) (end 33.2 93.65) (width 0.3) (layer "B.Cu") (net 3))
 (segment (start 24.95 94.8875) (end 24.6125 94.8875) (width 0.3) (layer "B.Cu") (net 3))
 (segment (start 30.55 96.1) (end 30.55 93.65) (width 0.3) (layer "B.Cu") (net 3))
 (segment (start 21.35 98.15) (end 21.35 99.1) (width 0.3) (layer "B.Cu") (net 3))
 (segment (start 28.95 94.7) (end 30 93.65) (width 0.3) (layer "B.Cu") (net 3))
 (segment (start 39.5 93.65) (end 40.875 95.025) (width 0.3) (layer "B.Cu") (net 3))
 (segment (start 30.1 96.55) (end 30.55 96.1) (width 0.3) (layer "B.Cu") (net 3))
 (segment (start 40.875 95.025) (end 40.875 98.65) (width 0.3) (layer "B.Cu") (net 3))
 (segment (start 30 93.65) (end 30.55 93.65) (width 0.3) (layer "B.Cu") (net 3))
 (segment (start 24.6125 94.8875) (end 21.35 98.15) (width 0.3) (layer "B.Cu") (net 3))
 (segment (start 37.85 92.9) (end 38.75 92.9) (width 0.3) (layer "B.Cu") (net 3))
 (segment (start 33 91.65) (end 33.8625 90.7875) (width 0.3) (layer "F.Cu") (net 1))
 (segment (start 31.4 97.4) (end 33 95.8) (width 0.3) (layer "F.Cu") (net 1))
 (segment (start 25.900431 99.1) (end 27.600431 97.4) (width 0.3) (layer "F.Cu") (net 1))
 (segment (start 35.95 87.8625) (end 35.95 90.7875) (width 0.3) (layer "F.Cu") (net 1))
 (segment (start 33.8625 90.7875) (end 35.95 90.7875) (width 0.3) (layer "F.Cu") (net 1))
 (segment (start 25.35 99.1) (end 25.900431 99.1) (width 0.3) (layer "F.Cu") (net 1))
 (segment (start 27.600431 97.4) (end 31.4 97.4) (width 0.3) (layer "F.Cu") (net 1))
 (segment (start 33 95.8) (end 33 91.65) (width 0.3) (layer "F.Cu") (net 1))
 (segment (start 42.4 82.05) (end 43.75 83.4) (width 0.3) (layer "F.Cu") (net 10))
 (segment (start 39.45 82.55) (end 40 82.55) (width 0.3) (layer "F.Cu") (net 10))
 (segment (start 40 82.55) (end 40.5 82.05) (width 0.3) (layer "F.Cu") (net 10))
 (segment (start 40.5 82.05) (end 42.4 82.05) (width 0.3) (layer "F.Cu") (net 10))
 (segment (start 43.75 83.4) (end 43.75 84.86) (width 0.3) (layer "F.Cu") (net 10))
 (via (at 39.45 82.55) (size 0.8) (drill 0.4) (layers "F.Cu" "B.Cu") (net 10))
 (segment (start 38.45 89.24) (end 38.037893 89.24) (width 0.3) (layer "B.Cu") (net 10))
 (segment (start 38.037893 89.24) (end 36.7 87.902107) (width 0.3) (layer "B.Cu") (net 10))
 (segment (start 36.7 87.902107) (end 36.7 85) (width 0.3) (layer "B.Cu") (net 10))
 (segment (start 39.15 82.55) (end 39.45 82.55) (width 0.3) (layer "B.Cu") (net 10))
 (segment (start 36.7 85) (end 39.15 82.55) (width 0.3) (layer "B.Cu") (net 10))
 (segment (start 43.75 95.02) (end 39.9425 91.2125) (width 0.3) (layer "F.Cu") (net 12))
 (segment (start 38.9 91.2125) (end 38.8625 91.2125) (width 0.3) (layer "F.Cu") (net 12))
 (segment (start 39.9425 91.2125) (end 38.9 91.2125) (width 0.3) (layer "F.Cu") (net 12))
 (segment (start 38.8625 91.2125) (end 36.75 89.1) (width 0.3) (layer "F.Cu") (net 12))
 (via (at 36.75 89.1) (size 0.8) (drill 0.4) (layers "F.Cu" "B.Cu") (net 12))
 (segment (start 36.75 89.1) (end 35.55 89.1) (width 0.3) (layer "B.Cu") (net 12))
 (segment (start 35.55 89.1) (end 34.42 87.97) (width 0.3) (layer "B.Cu") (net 12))
 (segment (start 34.42 87.97) (end 33.5 87.97) (width 0.3) (layer "B.Cu") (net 12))
 (segment (start 29.95 92.6) (end 29.1 93.45) (width 0.3) (layer "B.Cu") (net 14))
 (segment (start 27.05 94.7) (end 26.9625 94.7) (width 0.3) (layer "B.Cu") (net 14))
 (segment (start 25.7 82.385) (end 25.7 86.4) (width 0.3) (layer "B.Cu") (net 14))
 (segment (start 29.1 93.45) (end 27.75 93.45) (width 0.3) (layer "B.Cu") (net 14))
 (segment (start 27.05 94.15) (end 27.05 94.7) (width 0.3) (layer "B.Cu") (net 14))
 (segment (start 26.9625 94.7) (end 24.95 96.7125) (width 0.3) (layer "B.Cu") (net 14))
 (segment (start 27.75 93.45) (end 27.05 94.15) (width 0.3) (layer "B.Cu") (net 14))
 (segment (start 25.7 86.4) (end 29.95 90.65) (width 0.3) (layer "B.Cu") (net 14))
 (segment (start 29.95 90.65) (end 29.95 92.6) (width 0.3) (layer "B.Cu") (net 14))
 (segment (start 42.15 96.75) (end 41.4 96) (width 0.3) (layer "B.Cu") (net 15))
 (segment (start 41.4 91.2) (end 41.15 90.95) (width 0.3) (layer "B.Cu") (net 15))
 (segment (start 39 99.6) (end 41.65 99.6) (width 0.3) (layer "B.Cu") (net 15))
 (segment (start 41.65 99.6) (end 42.15 99.1) (width 0.3) (layer "B.Cu") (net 15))
 (segment (start 42.15 99.1) (end 42.15 96.75) (width 0.3) (layer "B.Cu") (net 15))
 (segment (start 41.15 90.95) (end 36.25 90.95) (width 0.3) (layer "B.Cu") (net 15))
 (segment (start 41.4 96) (end 41.4 91.2) (width 0.3) (layer "B.Cu") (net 15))
 (segment (start 34.54 89.24) (end 33.5 89.24) (width 0.3) (layer "B.Cu") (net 15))
 (segment (start 36.25 90.95) (end 34.54 89.24) (width 0.3) (layer "B.Cu") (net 15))
 (segment (start 23.4 94.35) (end 24.4 93.35) (width 0.3) (layer "B.Cu") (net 13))
 (segment (start 23.1125 94.35) (end 23.4 94.35) (width 0.3) (layer "B.Cu") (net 13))
 (segment (start 24.4 93.35) (end 26.805 93.35) (width 0.3) (layer "B.Cu") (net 13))
 (segment (start 26.805 93.35) (end 28.24 91.915) (width 0.3) (layer "B.Cu") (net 13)))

